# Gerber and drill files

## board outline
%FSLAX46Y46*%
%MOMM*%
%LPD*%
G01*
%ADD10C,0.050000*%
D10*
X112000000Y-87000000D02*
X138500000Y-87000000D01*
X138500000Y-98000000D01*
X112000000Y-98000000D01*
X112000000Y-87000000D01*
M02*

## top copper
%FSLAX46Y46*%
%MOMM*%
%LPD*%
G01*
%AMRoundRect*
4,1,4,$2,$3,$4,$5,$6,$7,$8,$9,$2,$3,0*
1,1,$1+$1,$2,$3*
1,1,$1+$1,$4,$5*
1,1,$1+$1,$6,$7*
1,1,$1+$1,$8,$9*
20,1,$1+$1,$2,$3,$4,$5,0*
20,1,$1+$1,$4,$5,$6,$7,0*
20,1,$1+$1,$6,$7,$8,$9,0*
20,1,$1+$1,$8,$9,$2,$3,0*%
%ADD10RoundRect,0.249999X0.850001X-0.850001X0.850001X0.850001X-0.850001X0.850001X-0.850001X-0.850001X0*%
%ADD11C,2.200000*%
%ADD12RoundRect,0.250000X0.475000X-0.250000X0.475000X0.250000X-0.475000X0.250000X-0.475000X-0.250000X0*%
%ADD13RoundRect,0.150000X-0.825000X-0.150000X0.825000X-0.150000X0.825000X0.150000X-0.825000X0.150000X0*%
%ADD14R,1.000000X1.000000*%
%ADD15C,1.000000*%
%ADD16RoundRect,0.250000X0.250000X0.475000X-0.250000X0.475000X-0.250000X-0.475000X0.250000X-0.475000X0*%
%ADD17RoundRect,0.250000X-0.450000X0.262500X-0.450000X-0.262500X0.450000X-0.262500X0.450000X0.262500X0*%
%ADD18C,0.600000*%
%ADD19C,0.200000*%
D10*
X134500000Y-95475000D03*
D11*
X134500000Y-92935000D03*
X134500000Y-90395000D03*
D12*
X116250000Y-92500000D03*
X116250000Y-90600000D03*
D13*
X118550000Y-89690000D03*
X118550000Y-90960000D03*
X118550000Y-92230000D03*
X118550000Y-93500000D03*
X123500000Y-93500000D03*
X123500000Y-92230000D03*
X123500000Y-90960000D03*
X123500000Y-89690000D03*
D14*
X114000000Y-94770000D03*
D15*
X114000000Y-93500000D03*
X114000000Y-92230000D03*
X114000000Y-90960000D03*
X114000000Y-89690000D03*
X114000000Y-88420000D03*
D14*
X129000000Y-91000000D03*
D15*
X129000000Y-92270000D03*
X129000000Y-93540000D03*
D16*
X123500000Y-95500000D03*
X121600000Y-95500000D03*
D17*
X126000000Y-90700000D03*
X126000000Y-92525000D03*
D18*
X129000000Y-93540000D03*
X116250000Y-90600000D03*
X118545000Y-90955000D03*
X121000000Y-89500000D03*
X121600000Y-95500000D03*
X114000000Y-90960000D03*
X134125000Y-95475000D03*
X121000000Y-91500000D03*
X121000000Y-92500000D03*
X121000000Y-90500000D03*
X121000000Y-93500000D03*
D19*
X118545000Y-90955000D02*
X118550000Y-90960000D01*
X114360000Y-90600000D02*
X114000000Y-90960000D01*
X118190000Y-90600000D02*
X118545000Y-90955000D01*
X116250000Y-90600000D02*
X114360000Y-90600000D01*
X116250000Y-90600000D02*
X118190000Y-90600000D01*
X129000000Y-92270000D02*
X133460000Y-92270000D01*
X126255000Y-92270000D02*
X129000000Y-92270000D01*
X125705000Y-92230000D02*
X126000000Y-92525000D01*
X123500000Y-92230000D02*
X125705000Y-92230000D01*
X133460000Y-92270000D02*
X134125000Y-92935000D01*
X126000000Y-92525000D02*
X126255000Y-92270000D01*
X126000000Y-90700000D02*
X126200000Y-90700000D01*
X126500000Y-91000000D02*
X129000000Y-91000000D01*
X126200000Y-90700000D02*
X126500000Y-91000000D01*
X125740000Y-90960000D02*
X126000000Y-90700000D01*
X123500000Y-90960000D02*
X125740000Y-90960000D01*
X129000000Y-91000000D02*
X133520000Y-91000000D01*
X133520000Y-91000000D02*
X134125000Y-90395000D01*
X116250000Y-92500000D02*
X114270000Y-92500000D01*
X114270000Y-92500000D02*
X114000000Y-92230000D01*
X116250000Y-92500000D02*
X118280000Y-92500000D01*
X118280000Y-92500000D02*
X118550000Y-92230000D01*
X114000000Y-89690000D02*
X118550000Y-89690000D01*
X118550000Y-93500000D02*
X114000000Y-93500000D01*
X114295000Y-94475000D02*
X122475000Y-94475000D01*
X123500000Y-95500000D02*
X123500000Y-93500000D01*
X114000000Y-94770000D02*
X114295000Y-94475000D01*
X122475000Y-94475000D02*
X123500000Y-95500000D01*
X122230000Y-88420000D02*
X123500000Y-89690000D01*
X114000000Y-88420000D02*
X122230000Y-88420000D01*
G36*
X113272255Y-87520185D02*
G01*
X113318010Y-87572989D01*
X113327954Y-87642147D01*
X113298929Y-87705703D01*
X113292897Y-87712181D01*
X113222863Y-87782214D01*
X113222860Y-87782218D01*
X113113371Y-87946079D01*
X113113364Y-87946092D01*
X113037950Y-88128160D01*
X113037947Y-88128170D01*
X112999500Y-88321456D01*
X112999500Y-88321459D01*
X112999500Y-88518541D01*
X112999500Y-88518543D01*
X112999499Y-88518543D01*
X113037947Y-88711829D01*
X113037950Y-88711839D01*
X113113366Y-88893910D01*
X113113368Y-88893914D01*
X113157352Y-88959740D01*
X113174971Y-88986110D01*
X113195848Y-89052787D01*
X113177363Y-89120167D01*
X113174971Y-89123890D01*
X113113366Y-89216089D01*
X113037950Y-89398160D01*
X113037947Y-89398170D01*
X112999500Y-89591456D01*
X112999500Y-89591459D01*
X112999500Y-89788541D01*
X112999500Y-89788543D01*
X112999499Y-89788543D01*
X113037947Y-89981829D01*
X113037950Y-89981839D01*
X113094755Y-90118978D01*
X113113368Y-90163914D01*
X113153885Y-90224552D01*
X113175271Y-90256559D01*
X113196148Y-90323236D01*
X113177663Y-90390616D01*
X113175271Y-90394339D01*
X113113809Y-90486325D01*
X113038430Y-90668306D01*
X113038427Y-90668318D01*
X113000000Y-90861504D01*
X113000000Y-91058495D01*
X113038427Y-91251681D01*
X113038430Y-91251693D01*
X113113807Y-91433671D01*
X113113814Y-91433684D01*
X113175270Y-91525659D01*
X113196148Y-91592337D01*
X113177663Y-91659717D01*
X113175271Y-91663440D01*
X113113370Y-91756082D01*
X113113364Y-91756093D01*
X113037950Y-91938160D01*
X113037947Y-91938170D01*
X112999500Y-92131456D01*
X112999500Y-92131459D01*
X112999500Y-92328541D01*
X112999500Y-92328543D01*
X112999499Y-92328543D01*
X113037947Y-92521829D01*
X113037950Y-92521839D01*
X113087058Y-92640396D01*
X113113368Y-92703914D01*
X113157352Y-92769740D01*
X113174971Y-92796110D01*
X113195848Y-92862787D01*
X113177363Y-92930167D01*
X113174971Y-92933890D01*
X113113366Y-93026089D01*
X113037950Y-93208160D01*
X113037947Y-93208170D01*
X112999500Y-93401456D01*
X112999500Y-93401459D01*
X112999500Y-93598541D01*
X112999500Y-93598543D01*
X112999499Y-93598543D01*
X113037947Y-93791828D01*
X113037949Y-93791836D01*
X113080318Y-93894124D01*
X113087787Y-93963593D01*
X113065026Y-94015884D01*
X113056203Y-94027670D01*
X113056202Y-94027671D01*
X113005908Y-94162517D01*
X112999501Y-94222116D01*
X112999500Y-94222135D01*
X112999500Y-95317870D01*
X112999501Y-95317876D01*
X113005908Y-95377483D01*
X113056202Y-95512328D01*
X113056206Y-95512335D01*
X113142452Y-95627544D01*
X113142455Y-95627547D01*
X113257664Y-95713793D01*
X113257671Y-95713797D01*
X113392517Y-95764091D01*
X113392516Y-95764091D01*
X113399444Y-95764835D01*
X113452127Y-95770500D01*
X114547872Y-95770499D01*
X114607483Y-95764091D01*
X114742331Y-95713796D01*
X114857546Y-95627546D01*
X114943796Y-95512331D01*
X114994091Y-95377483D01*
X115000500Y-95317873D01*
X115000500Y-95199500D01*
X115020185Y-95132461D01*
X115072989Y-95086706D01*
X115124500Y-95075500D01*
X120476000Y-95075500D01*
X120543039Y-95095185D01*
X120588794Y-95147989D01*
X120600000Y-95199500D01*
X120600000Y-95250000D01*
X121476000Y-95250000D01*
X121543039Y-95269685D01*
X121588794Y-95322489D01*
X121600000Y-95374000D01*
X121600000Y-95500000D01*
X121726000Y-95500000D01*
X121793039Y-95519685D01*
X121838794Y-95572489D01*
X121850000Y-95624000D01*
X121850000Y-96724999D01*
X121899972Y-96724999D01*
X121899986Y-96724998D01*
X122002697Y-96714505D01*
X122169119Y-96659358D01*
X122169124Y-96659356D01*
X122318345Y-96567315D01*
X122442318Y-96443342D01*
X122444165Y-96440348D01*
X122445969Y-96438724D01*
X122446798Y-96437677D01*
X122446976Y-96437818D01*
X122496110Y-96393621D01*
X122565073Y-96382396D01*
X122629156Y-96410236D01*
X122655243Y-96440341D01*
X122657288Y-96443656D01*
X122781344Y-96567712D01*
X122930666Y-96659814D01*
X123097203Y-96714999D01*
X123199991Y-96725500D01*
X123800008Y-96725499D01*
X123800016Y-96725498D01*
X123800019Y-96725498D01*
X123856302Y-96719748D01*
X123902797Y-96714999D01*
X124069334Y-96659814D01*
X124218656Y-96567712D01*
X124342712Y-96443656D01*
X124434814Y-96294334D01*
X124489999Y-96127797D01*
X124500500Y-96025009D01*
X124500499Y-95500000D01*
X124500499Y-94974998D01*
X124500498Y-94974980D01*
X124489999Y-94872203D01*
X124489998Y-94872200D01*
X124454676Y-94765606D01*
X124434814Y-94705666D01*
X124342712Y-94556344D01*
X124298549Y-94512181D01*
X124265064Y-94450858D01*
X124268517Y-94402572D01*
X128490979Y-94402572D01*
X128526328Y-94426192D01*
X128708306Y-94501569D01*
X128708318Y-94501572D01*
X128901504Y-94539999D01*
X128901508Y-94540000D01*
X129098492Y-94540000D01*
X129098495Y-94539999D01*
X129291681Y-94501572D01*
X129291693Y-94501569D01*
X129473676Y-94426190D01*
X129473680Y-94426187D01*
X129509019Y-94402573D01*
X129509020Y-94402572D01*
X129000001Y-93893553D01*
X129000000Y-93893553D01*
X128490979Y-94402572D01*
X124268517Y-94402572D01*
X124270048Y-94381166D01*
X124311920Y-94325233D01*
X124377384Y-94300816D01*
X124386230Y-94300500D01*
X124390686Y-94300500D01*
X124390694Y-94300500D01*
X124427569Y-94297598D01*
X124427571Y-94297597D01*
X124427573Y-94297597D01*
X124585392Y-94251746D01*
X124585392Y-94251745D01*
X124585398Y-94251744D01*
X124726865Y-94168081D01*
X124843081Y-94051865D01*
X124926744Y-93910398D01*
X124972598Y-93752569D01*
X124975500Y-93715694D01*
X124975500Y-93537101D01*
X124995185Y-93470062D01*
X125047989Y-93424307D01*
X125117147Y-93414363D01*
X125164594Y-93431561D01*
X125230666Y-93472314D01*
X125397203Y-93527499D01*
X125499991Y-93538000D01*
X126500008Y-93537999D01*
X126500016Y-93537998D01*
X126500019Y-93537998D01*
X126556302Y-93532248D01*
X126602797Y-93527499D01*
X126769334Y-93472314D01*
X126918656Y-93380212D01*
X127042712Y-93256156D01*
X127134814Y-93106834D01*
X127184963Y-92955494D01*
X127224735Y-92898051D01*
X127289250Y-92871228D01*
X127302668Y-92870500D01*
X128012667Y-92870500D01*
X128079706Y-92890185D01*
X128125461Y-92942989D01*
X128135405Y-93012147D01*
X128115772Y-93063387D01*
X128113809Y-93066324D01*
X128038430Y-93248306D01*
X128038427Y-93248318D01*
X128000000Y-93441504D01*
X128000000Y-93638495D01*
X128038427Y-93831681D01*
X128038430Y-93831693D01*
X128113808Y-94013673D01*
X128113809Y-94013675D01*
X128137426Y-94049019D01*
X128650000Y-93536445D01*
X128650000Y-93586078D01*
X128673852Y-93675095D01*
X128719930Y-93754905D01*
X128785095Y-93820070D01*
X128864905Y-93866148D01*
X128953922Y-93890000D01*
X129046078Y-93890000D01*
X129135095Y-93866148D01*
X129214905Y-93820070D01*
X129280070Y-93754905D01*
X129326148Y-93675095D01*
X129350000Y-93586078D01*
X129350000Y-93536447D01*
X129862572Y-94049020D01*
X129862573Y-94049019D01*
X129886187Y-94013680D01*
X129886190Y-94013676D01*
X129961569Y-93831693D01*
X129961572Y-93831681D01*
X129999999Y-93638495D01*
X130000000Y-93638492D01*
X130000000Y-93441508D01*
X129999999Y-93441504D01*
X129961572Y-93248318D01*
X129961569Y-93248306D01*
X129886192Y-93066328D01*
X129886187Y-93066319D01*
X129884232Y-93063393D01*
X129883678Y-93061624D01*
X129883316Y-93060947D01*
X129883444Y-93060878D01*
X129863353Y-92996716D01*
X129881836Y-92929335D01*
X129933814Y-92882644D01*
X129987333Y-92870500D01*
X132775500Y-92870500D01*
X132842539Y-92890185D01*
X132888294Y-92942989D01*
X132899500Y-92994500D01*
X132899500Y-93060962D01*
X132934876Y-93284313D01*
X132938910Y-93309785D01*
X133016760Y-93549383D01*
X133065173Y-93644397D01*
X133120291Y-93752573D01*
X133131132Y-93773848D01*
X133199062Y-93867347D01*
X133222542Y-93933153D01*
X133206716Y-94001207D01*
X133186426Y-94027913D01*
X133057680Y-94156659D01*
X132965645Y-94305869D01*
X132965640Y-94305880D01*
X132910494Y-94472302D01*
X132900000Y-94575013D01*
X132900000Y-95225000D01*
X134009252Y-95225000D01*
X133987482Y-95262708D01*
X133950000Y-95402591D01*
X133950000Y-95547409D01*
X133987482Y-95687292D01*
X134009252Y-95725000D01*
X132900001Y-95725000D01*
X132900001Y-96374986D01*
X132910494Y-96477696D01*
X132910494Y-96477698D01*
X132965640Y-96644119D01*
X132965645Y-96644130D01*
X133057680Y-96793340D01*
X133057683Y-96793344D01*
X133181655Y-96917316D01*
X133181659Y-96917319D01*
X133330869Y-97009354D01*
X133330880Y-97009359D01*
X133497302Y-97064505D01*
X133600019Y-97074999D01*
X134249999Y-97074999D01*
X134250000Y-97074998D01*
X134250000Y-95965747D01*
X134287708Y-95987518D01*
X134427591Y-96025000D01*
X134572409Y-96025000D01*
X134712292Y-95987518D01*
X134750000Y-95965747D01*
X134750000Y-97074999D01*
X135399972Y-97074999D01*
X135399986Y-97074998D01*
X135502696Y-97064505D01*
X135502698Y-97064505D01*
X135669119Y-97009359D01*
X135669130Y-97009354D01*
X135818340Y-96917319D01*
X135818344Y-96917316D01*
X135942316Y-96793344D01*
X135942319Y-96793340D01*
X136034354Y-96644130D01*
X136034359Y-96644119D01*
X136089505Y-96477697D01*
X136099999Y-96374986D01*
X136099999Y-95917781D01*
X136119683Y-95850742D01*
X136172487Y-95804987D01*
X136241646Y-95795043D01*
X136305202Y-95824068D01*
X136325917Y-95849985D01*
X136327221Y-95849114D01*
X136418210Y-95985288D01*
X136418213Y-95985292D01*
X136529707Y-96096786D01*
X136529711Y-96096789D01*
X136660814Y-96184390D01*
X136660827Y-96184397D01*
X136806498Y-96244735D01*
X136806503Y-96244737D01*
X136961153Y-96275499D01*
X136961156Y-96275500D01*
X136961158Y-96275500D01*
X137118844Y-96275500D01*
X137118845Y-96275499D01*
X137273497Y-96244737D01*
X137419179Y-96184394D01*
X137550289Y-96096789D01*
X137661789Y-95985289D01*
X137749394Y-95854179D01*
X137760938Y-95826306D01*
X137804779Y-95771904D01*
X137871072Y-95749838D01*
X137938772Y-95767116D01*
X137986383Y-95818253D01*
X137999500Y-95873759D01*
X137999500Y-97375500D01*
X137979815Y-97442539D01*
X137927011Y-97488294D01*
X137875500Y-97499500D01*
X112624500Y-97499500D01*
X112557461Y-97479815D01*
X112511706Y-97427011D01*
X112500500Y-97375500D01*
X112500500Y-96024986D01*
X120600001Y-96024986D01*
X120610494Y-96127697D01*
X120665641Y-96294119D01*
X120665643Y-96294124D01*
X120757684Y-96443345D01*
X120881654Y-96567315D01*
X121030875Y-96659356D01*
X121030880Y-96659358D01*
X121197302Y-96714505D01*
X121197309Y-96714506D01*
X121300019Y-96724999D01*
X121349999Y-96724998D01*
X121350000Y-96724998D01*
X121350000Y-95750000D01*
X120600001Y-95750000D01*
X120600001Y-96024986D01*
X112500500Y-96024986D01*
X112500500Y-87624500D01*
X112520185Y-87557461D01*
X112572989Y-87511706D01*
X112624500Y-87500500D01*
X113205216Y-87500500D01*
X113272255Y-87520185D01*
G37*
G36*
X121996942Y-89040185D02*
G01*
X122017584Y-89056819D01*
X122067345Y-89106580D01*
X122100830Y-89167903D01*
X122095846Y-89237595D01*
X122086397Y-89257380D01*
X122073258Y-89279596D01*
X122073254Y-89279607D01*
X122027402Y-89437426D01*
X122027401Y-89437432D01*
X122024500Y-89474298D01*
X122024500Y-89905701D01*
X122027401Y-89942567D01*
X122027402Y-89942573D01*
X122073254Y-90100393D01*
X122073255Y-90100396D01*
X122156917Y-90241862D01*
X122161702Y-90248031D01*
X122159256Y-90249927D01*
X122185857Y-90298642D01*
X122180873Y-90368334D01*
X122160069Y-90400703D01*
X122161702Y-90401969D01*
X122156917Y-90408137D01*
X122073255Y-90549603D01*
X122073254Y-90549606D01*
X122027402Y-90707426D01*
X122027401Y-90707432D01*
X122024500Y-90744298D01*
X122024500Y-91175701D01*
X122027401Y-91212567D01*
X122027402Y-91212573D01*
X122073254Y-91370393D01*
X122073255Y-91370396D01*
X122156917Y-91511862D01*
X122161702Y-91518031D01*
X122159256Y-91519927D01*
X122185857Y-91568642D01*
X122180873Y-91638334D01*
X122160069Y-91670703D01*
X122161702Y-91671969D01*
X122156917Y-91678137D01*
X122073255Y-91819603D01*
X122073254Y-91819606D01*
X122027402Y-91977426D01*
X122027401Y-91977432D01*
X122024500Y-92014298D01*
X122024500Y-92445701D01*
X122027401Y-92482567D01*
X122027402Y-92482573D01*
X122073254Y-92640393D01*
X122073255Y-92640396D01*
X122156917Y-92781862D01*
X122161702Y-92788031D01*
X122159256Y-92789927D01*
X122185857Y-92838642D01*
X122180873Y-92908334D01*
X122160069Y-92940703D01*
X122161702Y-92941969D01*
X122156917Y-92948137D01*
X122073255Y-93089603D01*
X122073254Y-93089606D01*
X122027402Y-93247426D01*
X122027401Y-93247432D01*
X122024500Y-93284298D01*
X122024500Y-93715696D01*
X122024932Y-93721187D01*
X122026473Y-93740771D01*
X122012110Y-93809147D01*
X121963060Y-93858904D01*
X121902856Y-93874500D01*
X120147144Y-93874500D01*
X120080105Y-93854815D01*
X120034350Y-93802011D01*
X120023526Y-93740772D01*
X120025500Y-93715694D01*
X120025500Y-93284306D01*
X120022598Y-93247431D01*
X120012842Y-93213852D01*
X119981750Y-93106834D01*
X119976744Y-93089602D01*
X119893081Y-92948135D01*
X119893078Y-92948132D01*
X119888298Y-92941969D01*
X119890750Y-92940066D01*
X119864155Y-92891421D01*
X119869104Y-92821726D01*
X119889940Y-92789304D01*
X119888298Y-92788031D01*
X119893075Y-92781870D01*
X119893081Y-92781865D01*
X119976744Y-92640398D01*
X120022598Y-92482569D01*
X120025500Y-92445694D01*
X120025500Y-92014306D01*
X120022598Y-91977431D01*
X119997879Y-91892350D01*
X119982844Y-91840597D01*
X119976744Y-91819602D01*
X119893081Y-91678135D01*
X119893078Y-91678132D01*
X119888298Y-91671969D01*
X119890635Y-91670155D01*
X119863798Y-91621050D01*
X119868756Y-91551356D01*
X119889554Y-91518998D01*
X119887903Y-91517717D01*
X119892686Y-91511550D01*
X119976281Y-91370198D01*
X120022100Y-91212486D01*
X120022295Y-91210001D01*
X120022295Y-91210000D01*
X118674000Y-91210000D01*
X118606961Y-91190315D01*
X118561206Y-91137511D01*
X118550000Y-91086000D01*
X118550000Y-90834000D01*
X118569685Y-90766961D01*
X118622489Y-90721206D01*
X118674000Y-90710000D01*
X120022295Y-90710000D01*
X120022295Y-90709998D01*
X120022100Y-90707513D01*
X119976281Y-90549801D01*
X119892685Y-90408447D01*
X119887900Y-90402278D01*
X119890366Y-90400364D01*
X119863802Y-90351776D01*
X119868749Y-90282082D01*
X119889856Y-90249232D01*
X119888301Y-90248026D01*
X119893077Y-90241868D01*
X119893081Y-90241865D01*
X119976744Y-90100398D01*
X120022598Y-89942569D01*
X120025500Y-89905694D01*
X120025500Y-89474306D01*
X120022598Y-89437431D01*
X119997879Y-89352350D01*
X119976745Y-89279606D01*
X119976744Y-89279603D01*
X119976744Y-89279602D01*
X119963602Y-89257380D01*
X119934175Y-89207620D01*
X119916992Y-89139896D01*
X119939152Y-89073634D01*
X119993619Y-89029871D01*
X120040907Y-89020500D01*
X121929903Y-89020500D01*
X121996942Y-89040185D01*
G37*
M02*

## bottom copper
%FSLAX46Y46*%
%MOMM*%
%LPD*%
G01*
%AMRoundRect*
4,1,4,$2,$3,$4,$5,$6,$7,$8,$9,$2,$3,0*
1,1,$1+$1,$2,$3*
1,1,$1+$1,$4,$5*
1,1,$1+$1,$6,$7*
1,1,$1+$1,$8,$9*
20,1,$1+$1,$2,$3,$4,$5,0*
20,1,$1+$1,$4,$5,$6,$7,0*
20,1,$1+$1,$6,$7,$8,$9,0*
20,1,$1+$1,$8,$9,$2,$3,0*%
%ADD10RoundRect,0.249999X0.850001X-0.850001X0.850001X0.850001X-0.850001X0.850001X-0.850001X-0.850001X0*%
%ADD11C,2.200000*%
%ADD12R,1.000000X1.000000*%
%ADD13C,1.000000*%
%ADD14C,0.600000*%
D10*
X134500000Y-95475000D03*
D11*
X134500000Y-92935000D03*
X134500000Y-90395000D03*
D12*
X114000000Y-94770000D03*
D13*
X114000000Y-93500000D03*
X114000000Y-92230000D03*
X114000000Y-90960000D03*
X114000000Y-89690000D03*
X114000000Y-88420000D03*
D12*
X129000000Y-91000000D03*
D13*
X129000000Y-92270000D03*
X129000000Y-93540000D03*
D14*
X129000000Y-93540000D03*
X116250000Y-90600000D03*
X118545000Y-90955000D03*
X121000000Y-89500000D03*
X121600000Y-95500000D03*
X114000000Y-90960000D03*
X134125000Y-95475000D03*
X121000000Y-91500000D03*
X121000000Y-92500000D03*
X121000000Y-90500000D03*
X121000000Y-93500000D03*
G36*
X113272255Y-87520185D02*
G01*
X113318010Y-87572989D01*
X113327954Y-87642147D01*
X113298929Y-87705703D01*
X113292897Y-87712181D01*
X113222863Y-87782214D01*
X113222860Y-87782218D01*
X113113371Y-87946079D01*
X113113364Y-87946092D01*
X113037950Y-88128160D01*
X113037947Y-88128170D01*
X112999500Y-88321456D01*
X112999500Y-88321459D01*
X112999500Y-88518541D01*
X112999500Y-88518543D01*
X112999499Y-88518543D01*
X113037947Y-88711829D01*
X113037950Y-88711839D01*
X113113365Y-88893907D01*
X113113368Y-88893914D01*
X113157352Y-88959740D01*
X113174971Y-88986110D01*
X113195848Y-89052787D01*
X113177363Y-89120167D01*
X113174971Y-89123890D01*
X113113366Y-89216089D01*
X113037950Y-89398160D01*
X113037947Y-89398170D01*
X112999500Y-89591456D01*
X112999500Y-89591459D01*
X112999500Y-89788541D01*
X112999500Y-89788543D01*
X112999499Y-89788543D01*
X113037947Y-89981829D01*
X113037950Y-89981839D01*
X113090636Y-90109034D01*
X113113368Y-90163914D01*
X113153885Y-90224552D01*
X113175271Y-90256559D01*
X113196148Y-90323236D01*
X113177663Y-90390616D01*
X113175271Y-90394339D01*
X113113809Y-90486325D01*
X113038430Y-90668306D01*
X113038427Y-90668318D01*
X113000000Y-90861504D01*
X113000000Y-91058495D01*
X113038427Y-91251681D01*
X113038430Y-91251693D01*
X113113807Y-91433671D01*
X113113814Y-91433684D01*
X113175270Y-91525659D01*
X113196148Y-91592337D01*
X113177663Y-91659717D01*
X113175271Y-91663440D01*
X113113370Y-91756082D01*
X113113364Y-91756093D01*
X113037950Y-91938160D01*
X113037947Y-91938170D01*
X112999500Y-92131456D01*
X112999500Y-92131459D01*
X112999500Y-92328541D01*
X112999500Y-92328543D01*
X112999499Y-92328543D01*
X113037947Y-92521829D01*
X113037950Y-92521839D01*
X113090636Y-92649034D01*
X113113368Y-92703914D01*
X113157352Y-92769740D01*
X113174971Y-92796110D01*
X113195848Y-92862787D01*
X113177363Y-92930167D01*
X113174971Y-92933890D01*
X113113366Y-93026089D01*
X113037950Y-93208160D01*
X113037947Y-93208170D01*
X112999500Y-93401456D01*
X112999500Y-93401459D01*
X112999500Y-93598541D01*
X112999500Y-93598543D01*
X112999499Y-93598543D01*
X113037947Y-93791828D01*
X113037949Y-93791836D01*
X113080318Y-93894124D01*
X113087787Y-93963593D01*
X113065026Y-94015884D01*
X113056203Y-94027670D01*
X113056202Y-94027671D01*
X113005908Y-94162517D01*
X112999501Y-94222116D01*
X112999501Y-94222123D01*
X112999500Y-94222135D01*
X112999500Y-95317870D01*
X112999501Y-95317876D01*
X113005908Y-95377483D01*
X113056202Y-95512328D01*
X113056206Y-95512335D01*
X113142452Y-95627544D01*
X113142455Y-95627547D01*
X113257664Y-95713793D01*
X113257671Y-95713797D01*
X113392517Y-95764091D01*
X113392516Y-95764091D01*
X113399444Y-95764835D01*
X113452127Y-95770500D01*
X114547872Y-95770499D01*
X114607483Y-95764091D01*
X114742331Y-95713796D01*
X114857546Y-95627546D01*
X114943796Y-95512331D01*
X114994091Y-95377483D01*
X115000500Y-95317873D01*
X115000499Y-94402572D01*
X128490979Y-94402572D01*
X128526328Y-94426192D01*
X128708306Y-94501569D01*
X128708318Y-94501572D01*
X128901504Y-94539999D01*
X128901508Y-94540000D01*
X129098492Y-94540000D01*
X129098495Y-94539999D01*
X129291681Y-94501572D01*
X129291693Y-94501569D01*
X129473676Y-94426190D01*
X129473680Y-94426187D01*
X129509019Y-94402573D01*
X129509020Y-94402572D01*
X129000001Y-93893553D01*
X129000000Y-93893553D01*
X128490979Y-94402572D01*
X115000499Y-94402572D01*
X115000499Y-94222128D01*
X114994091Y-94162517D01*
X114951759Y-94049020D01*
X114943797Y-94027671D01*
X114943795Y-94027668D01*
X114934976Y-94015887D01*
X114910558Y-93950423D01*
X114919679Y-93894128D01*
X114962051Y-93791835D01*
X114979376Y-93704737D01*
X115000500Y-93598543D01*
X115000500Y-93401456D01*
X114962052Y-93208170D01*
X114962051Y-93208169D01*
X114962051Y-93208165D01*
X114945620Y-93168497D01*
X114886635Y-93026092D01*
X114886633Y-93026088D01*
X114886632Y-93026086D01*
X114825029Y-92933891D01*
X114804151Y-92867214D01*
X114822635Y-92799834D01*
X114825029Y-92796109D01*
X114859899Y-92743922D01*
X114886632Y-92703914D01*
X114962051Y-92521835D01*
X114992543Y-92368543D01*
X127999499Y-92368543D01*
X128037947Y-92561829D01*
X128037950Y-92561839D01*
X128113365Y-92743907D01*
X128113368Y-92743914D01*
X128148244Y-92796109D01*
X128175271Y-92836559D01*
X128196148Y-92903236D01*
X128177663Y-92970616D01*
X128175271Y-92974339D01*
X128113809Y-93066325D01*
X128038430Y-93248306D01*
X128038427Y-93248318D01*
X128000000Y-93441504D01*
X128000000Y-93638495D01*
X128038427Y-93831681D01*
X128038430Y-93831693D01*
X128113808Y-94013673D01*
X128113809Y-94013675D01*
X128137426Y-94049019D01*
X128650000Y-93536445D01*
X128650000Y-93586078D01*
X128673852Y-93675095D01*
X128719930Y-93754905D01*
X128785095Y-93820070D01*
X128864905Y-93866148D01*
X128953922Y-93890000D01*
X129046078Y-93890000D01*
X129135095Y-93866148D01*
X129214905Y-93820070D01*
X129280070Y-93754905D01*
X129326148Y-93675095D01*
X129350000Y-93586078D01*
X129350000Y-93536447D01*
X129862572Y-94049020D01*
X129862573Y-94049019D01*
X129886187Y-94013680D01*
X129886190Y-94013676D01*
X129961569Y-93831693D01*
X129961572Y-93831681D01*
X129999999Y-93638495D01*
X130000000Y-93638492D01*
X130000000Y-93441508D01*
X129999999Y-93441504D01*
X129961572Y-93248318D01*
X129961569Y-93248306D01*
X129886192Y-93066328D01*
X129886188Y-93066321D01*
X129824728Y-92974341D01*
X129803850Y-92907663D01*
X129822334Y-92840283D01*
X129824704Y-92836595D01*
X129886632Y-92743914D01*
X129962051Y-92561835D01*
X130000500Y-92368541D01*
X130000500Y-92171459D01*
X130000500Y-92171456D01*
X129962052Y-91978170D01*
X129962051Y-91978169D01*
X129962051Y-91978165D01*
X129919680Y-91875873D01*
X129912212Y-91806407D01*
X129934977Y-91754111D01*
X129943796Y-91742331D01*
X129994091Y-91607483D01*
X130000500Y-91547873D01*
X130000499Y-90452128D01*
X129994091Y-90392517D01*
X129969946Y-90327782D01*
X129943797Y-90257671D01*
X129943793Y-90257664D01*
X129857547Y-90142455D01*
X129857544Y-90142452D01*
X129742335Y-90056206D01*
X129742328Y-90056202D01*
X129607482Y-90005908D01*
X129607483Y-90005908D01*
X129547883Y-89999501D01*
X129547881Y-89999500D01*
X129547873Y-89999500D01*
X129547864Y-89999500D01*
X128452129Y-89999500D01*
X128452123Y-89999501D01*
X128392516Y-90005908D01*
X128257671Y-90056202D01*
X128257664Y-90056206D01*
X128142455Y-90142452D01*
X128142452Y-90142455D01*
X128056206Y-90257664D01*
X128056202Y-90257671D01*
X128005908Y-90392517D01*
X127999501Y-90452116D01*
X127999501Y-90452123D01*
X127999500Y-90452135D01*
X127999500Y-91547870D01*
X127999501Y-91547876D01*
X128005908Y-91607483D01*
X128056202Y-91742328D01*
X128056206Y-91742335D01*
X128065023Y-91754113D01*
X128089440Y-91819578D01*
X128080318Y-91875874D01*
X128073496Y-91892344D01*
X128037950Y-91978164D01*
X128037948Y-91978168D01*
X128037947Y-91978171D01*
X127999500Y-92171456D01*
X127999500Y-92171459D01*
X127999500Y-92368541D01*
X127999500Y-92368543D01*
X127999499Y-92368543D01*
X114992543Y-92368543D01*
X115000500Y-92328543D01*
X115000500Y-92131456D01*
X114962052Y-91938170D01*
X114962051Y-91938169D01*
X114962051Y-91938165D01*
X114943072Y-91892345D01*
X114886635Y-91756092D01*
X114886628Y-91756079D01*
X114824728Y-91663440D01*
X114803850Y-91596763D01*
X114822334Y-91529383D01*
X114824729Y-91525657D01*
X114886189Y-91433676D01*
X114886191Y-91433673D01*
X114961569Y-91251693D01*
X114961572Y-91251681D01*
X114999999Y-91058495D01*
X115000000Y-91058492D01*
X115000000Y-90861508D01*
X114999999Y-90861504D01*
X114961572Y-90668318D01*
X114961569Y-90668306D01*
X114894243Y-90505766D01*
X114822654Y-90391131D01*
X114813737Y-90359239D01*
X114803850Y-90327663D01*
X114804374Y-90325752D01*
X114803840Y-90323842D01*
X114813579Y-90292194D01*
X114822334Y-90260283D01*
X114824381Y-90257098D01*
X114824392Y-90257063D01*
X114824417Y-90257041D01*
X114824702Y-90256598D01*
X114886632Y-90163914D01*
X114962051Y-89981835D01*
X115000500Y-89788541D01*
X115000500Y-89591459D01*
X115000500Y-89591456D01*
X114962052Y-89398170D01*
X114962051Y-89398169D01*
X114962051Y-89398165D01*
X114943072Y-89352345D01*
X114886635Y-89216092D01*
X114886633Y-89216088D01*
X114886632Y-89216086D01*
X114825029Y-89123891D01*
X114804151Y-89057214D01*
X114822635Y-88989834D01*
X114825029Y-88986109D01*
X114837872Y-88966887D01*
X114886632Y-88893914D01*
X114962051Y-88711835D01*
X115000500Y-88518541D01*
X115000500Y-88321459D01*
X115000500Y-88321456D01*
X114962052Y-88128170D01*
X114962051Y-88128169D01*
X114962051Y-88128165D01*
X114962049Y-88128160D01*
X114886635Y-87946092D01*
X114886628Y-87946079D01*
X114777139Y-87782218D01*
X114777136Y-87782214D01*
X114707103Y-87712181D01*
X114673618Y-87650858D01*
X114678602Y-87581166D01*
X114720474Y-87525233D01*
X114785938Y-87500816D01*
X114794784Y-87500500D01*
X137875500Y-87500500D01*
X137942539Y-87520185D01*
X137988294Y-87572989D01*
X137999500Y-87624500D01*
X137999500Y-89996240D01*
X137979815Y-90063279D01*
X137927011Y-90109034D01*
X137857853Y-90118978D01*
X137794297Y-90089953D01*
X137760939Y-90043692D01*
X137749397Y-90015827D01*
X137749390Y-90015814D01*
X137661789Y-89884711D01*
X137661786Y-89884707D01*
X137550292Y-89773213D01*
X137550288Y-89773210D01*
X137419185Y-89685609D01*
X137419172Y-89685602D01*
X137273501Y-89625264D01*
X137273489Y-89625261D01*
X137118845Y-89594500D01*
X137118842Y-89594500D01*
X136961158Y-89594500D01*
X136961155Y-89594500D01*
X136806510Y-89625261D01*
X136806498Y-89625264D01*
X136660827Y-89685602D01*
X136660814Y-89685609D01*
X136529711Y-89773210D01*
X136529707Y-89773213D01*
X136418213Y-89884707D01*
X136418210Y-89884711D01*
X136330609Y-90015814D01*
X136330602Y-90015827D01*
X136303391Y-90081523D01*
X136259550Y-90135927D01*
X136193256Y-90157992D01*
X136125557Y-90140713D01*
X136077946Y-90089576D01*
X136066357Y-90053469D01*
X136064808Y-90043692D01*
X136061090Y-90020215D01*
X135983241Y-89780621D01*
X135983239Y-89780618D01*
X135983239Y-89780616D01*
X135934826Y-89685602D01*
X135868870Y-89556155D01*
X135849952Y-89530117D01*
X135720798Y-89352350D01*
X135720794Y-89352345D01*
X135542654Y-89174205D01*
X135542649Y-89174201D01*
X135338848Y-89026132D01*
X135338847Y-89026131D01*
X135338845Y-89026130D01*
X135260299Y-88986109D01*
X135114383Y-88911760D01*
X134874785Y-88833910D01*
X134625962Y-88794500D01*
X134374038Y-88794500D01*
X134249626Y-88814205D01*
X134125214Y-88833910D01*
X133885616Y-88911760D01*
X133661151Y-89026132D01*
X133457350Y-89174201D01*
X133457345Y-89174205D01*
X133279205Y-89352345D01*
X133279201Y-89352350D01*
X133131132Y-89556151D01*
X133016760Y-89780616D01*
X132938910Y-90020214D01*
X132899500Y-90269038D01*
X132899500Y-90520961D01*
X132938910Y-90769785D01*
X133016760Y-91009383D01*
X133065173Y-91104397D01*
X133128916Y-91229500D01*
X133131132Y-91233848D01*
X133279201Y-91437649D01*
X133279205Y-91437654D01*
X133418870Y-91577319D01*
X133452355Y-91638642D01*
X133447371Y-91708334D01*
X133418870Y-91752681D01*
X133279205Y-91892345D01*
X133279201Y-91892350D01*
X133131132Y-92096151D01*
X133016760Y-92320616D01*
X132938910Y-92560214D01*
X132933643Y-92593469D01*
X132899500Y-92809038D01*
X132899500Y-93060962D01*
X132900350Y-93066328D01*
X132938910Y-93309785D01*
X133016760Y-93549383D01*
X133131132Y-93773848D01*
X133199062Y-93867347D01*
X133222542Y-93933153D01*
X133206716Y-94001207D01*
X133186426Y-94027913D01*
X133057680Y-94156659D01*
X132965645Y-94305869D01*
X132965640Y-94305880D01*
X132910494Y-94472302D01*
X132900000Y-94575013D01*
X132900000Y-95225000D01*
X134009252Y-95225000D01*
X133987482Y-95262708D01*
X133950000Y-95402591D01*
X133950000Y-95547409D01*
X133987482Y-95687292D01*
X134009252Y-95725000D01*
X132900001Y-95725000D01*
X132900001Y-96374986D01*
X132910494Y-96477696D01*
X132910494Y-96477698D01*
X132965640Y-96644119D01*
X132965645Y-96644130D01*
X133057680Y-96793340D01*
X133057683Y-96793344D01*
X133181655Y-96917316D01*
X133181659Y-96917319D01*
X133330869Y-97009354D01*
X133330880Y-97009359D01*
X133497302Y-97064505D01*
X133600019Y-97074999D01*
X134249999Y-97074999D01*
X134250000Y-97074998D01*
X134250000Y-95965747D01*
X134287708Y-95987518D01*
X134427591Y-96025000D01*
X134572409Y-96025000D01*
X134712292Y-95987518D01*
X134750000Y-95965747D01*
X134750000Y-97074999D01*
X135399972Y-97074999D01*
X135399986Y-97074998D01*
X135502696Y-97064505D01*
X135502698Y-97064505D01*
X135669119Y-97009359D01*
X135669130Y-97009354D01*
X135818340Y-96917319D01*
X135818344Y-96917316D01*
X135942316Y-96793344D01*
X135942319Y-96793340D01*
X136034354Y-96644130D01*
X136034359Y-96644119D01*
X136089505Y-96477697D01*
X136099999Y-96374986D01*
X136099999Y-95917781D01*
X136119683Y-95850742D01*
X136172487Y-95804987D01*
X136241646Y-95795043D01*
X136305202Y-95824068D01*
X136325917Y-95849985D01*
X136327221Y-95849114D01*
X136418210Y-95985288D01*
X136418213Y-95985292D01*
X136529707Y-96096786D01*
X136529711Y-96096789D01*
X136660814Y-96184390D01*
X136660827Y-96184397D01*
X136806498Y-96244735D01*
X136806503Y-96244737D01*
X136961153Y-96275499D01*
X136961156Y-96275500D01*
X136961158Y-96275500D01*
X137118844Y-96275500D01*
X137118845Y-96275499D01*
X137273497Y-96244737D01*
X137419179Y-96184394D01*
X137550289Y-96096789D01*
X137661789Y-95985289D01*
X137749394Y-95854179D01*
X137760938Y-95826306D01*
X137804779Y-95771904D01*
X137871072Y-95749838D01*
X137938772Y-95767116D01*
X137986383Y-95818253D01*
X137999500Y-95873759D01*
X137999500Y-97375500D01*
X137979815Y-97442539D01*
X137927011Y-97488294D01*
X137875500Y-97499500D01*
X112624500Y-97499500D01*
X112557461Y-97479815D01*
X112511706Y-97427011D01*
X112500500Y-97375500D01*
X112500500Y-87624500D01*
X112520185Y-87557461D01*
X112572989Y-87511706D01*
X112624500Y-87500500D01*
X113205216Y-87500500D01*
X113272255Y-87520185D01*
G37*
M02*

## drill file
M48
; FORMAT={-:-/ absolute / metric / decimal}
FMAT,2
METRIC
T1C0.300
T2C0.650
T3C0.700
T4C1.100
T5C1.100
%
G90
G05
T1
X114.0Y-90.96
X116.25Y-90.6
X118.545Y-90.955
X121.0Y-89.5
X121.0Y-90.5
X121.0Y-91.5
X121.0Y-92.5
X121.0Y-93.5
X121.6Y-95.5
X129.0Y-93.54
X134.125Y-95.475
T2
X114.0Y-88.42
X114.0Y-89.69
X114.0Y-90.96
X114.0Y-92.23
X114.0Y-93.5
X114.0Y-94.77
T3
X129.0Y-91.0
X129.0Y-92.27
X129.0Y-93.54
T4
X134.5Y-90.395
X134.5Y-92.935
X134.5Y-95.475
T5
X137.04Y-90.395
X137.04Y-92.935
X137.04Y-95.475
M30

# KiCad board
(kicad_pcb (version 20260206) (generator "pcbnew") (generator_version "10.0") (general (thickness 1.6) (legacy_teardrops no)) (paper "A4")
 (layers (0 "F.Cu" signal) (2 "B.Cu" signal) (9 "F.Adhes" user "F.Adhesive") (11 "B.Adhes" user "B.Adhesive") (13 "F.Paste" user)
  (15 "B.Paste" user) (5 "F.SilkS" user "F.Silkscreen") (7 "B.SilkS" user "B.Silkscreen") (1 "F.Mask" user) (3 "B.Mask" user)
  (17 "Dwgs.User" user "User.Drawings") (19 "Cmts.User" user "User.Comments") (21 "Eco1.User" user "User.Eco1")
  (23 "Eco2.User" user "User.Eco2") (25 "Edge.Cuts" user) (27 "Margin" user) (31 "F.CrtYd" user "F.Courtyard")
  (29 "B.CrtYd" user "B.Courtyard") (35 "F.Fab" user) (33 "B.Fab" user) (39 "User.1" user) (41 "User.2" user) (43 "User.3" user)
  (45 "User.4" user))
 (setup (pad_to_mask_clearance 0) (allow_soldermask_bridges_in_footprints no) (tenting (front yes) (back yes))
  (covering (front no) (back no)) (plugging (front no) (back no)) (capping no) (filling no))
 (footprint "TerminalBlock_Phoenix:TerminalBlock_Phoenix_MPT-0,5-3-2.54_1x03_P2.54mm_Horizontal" (layer "F.Cu") (at 134.5 95.475 90)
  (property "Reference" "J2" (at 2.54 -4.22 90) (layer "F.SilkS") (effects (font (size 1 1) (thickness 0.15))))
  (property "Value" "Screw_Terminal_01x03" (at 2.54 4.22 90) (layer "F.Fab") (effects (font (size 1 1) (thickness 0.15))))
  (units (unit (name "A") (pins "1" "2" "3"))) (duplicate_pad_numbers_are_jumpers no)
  (pad "" np_thru_hole circle (at 0 2.54 90) (size 1.1 1.1) (drill 1.1) (layers "*.Cu" "*.Mask"))
  (pad "" np_thru_hole circle (at 2.54 2.54 90) (size 1.1 1.1) (drill 1.1) (layers "*.Cu" "*.Mask"))
  (pad "" np_thru_hole circle (at 5.08 2.54 90) (size 1.1 1.1) (drill 1.1) (layers "*.Cu" "*.Mask"))
  (pad "1" thru_hole roundrect (at 0 0 90) (size 2.2 2.2) (drill 1.1) (layers "*.Cu" "*.Mask") (remove_unused_layers no)
   (roundrect_rratio 0.113636) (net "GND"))
  (pad "2" thru_hole circle (at 2.54 0 90) (size 2.2 2.2) (drill 1.1) (layers "*.Cu" "*.Mask") (remove_unused_layers no) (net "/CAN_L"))
  (pad "3" thru_hole circle (at 5.08 0 90) (size 2.2 2.2) (drill 1.1) (layers "*.Cu" "*.Mask") (remove_unused_layers no) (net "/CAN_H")))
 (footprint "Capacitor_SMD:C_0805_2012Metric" (layer "F.Cu") (at 116.25 91.55 90)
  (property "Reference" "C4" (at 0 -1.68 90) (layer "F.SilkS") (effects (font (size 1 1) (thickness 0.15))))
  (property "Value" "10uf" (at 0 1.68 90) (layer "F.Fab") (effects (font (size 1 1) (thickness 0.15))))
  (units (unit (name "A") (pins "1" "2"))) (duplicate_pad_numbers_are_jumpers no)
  (pad "1" smd roundrect (at -0.95 0 90) (size 1 1.45) (layers "F.Cu" "F.Mask" "F.Paste") (roundrect_rratio 0.25) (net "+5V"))
  (pad "2" smd roundrect (at 0.95 0 90) (size 1 1.45) (layers "F.Cu" "F.Mask" "F.Paste") (roundrect_rratio 0.25) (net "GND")))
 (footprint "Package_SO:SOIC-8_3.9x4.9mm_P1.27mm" (layer "F.Cu") (at 121.025 91.595)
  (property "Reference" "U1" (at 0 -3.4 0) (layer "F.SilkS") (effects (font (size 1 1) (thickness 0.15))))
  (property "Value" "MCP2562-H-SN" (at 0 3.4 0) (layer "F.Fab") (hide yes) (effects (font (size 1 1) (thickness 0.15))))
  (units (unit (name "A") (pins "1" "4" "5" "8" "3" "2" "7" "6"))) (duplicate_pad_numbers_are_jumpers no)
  (pad "1" smd roundrect (at -2.475 -1.905) (size 1.95 0.6) (layers "F.Cu" "F.Mask" "F.Paste") (roundrect_rratio 0.25) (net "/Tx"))
  (pad "2" smd roundrect (at -2.475 -0.635) (size 1.95 0.6) (layers "F.Cu" "F.Mask" "F.Paste") (roundrect_rratio 0.25) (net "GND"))
  (pad "3" smd roundrect (at -2.475 0.635) (size 1.95 0.6) (layers "F.Cu" "F.Mask" "F.Paste") (roundrect_rratio 0.25) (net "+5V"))
  (pad "4" smd roundrect (at -2.475 1.905) (size 1.95 0.6) (layers "F.Cu" "F.Mask" "F.Paste") (roundrect_rratio 0.25) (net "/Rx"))
  (pad "5" smd roundrect (at 2.475 1.905) (size 1.95 0.6) (layers "F.Cu" "F.Mask" "F.Paste") (roundrect_rratio 0.25) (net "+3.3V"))
  (pad "6" smd roundrect (at 2.475 0.635) (size 1.95 0.6) (layers "F.Cu" "F.Mask" "F.Paste") (roundrect_rratio 0.25) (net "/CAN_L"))
  (pad "7" smd roundrect (at 2.475 -0.635) (size 1.95 0.6) (layers "F.Cu" "F.Mask" "F.Paste") (roundrect_rratio 0.25) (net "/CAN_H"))
  (pad "8" smd roundrect (at 2.475 -1.905) (size 1.95 0.6) (layers "F.Cu" "F.Mask" "F.Paste") (roundrect_rratio 0.25) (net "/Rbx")))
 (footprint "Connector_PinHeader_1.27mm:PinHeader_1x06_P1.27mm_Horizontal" (layer "F.Cu") (at 114 94.77 180)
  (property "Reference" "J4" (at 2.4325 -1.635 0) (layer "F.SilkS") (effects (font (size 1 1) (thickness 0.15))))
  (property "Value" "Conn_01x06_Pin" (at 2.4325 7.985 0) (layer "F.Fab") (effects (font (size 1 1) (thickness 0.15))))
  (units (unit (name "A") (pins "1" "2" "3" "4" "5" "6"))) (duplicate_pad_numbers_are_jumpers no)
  (pad "1" thru_hole rect (at 0 0 180) (size 1 1) (drill 0.65) (layers "*.Cu" "*.Mask") (remove_unused_layers no) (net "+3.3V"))
  (pad "2" thru_hole circle (at 0 1.27 180) (size 1 1) (drill 0.65) (layers "*.Cu" "*.Mask") (remove_unused_layers no) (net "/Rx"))
  (pad "3" thru_hole circle (at 0 2.54 180) (size 1 1) (drill 0.65) (layers "*.Cu" "*.Mask") (remove_unused_layers no) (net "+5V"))
  (pad "4" thru_hole circle (at 0 3.81 180) (size 1 1) (drill 0.65) (layers "*.Cu" "*.Mask") (remove_unused_layers no) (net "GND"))
  (pad "5" thru_hole circle (at 0 5.08 180) (size 1 1) (drill 0.65) (layers "*.Cu" "*.Mask") (remove_unused_layers no) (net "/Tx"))
  (pad "6" thru_hole circle (at 0 6.35 180) (size 1 1) (drill 0.65) (layers "*.Cu" "*.Mask") (remove_unused_layers no) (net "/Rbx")))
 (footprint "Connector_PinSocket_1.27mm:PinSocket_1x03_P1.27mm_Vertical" (layer "F.Cu") (at 129 91)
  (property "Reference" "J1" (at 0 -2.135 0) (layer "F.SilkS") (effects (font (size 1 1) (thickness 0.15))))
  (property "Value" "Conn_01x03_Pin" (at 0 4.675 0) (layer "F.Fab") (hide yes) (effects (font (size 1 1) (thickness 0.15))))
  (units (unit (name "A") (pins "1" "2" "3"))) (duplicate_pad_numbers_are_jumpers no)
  (pad "1" thru_hole rect (at 0 0) (size 1 1) (drill 0.7) (layers "*.Cu" "*.Mask") (remove_unused_layers no) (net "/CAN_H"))
  (pad "2" thru_hole circle (at 0 1.27) (size 1 1) (drill 0.7) (layers "*.Cu" "*.Mask") (remove_unused_layers no) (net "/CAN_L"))
  (pad "3" thru_hole circle (at 0 2.54) (size 1 1) (drill 0.7) (layers "*.Cu" "*.Mask") (remove_unused_layers no) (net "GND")))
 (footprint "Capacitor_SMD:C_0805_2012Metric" (layer "F.Cu") (at 122.55 95.5 180)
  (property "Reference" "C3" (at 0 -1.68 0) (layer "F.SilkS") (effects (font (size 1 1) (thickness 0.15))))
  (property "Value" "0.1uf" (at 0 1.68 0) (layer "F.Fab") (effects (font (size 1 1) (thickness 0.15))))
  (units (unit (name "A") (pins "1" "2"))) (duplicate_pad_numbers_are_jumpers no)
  (pad "1" smd roundrect (at -0.95 0 180) (size 1 1.45) (layers "F.Cu" "F.Mask" "F.Paste") (roundrect_rratio 0.25) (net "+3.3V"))
  (pad "2" smd roundrect (at 0.95 0 180) (size 1 1.45) (layers "F.Cu" "F.Mask" "F.Paste") (roundrect_rratio 0.25) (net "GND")))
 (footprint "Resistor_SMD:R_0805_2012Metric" (layer "F.Cu") (at 126 91.6125 -90)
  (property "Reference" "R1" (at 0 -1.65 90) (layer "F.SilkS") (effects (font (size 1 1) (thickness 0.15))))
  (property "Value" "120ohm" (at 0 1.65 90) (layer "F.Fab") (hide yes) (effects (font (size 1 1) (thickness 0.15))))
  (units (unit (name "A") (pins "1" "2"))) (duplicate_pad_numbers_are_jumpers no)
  (pad "1" smd roundrect (at -0.9125 0 270) (size 1.025 1.4) (layers "F.Cu" "F.Mask" "F.Paste") (roundrect_rratio 0.243902) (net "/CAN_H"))
  (pad "2" smd roundrect (at 0.9125 0 270) (size 1.025 1.4) (layers "F.Cu" "F.Mask" "F.Paste") (roundrect_rratio 0.243902) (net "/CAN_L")))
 (gr_rect (start 112 87) (end 138.5 98) (stroke (width 0.05) (type default)) (fill no) (layer "Edge.Cuts"))
 (segment (start 118.545 90.955) (end 118.55 90.96) (width 0.2) (layer "F.Cu") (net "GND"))
 (segment (start 114.36 90.6) (end 114 90.96) (width 0.2) (layer "F.Cu") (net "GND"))
 (segment (start 118.19 90.6) (end 118.545 90.955) (width 0.2) (layer "F.Cu") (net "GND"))
 (segment (start 116.25 90.6) (end 114.36 90.6) (width 0.2) (layer "F.Cu") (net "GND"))
 (segment (start 116.25 90.6) (end 118.19 90.6) (width 0.2) (layer "F.Cu") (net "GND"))
 (via (at 129 93.54) (size 0.6) (drill 0.3) (layers "F.Cu" "B.Cu") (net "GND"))
 (via (at 116.25 90.6) (size 0.6) (drill 0.3) (layers "F.Cu" "B.Cu") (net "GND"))
 (via (at 118.545 90.955) (size 0.6) (drill 0.3) (layers "F.Cu" "B.Cu") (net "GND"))
 (via (at 121 89.5) (size 0.6) (drill 0.3) (layers "F.Cu" "B.Cu") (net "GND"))
 (via (at 121.6 95.5) (size 0.6) (drill 0.3) (layers "F.Cu" "B.Cu") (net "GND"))
 (via (at 114 90.96) (size 0.6) (drill 0.3) (layers "F.Cu" "B.Cu") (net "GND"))
 (via (at 134.125 95.475) (size 0.6) (drill 0.3) (layers "F.Cu" "B.Cu") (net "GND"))
 (via (at 121 91.5) (size 0.6) (drill 0.3) (layers "F.Cu" "B.Cu") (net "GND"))
 (via (at 121 92.5) (size 0.6) (drill 0.3) (layers "F.Cu" "B.Cu") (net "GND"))
 (via (at 121 90.5) (size 0.6) (drill 0.3) (layers "F.Cu" "B.Cu") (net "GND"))
 (via (at 121 93.5) (size 0.6) (drill 0.3) (layers "F.Cu" "B.Cu") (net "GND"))
 (segment (start 129 92.27) (end 133.46 92.27) (width 0.2) (layer "F.Cu") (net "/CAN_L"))
 (segment (start 126.255 92.27) (end 129 92.27) (width 0.2) (layer "F.Cu") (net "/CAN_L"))
 (segment (start 125.705 92.23) (end 126 92.525) (width 0.2) (layer "F.Cu") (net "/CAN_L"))
 (segment (start 123.5 92.23) (end 125.705 92.23) (width 0.2) (layer "F.Cu") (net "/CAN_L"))
 (segment (start 133.46 92.27) (end 134.125 92.935) (width 0.2) (layer "F.Cu") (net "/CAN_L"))
 (segment (start 126 92.525) (end 126.255 92.27) (width 0.2) (layer "F.Cu") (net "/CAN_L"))
 (segment (start 126 90.7) (end 126.2 90.7) (width 0.2) (layer "F.Cu") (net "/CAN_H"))
 (segment (start 126.5 91) (end 129 91) (width 0.2) (layer "F.Cu") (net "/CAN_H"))
 (segment (start 126.2 90.7) (end 126.5 91) (width 0.2) (layer "F.Cu") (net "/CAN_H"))
 (segment (start 125.74 90.96) (end 126 90.7) (width 0.2) (layer "F.Cu") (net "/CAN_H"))
 (segment (start 123.5 90.96) (end 125.74 90.96) (width 0.2) (layer "F.Cu") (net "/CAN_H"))
 (segment (start 129 91) (end 133.52 91) (width 0.2) (layer "F.Cu") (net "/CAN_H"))
 (segment (start 133.52 91) (end 134.125 90.395) (width 0.2) (layer "F.Cu") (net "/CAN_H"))
 (segment (start 116.25 92.5) (end 114.27 92.5) (width 0.2) (layer "F.Cu") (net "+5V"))
 (segment (start 114.27 92.5) (end 114 92.23) (width 0.2) (layer "F.Cu") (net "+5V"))
 (segment (start 116.25 92.5) (end 118.28 92.5) (width 0.2) (layer "F.Cu") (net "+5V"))
 (segment (start 118.28 92.5) (end 118.55 92.23) (width 0.2) (layer "F.Cu") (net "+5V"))
 (segment (start 114 89.69) (end 118.55 89.69) (width 0.2) (layer "F.Cu") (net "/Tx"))
 (segment (start 118.55 93.5) (end 114 93.5) (width 0.2) (layer "F.Cu") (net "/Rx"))
 (segment (start 114.295 94.475) (end 122.475 94.475) (width 0.2) (layer "F.Cu") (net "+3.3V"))
 (segment (start 123.5 95.5) (end 123.5 93.5) (width 0.2) (layer "F.Cu") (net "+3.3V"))
 (segment (start 114 94.77) (end 114.295 94.475) (width 0.2) (layer "F.Cu") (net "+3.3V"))
 (segment (start 122.475 94.475) (end 123.5 95.5) (width 0.2) (layer "F.Cu") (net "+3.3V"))
 (segment (start 122.23 88.42) (end 123.5 89.69) (width 0.2) (layer "F.Cu") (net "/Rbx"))
 (segment (start 114 88.42) (end 122.23 88.42) (width 0.2) (layer "F.Cu") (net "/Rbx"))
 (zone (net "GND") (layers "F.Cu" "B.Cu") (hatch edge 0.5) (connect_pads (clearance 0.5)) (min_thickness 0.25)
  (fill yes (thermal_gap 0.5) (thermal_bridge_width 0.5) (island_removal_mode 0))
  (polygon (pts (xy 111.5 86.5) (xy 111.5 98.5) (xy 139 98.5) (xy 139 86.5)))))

